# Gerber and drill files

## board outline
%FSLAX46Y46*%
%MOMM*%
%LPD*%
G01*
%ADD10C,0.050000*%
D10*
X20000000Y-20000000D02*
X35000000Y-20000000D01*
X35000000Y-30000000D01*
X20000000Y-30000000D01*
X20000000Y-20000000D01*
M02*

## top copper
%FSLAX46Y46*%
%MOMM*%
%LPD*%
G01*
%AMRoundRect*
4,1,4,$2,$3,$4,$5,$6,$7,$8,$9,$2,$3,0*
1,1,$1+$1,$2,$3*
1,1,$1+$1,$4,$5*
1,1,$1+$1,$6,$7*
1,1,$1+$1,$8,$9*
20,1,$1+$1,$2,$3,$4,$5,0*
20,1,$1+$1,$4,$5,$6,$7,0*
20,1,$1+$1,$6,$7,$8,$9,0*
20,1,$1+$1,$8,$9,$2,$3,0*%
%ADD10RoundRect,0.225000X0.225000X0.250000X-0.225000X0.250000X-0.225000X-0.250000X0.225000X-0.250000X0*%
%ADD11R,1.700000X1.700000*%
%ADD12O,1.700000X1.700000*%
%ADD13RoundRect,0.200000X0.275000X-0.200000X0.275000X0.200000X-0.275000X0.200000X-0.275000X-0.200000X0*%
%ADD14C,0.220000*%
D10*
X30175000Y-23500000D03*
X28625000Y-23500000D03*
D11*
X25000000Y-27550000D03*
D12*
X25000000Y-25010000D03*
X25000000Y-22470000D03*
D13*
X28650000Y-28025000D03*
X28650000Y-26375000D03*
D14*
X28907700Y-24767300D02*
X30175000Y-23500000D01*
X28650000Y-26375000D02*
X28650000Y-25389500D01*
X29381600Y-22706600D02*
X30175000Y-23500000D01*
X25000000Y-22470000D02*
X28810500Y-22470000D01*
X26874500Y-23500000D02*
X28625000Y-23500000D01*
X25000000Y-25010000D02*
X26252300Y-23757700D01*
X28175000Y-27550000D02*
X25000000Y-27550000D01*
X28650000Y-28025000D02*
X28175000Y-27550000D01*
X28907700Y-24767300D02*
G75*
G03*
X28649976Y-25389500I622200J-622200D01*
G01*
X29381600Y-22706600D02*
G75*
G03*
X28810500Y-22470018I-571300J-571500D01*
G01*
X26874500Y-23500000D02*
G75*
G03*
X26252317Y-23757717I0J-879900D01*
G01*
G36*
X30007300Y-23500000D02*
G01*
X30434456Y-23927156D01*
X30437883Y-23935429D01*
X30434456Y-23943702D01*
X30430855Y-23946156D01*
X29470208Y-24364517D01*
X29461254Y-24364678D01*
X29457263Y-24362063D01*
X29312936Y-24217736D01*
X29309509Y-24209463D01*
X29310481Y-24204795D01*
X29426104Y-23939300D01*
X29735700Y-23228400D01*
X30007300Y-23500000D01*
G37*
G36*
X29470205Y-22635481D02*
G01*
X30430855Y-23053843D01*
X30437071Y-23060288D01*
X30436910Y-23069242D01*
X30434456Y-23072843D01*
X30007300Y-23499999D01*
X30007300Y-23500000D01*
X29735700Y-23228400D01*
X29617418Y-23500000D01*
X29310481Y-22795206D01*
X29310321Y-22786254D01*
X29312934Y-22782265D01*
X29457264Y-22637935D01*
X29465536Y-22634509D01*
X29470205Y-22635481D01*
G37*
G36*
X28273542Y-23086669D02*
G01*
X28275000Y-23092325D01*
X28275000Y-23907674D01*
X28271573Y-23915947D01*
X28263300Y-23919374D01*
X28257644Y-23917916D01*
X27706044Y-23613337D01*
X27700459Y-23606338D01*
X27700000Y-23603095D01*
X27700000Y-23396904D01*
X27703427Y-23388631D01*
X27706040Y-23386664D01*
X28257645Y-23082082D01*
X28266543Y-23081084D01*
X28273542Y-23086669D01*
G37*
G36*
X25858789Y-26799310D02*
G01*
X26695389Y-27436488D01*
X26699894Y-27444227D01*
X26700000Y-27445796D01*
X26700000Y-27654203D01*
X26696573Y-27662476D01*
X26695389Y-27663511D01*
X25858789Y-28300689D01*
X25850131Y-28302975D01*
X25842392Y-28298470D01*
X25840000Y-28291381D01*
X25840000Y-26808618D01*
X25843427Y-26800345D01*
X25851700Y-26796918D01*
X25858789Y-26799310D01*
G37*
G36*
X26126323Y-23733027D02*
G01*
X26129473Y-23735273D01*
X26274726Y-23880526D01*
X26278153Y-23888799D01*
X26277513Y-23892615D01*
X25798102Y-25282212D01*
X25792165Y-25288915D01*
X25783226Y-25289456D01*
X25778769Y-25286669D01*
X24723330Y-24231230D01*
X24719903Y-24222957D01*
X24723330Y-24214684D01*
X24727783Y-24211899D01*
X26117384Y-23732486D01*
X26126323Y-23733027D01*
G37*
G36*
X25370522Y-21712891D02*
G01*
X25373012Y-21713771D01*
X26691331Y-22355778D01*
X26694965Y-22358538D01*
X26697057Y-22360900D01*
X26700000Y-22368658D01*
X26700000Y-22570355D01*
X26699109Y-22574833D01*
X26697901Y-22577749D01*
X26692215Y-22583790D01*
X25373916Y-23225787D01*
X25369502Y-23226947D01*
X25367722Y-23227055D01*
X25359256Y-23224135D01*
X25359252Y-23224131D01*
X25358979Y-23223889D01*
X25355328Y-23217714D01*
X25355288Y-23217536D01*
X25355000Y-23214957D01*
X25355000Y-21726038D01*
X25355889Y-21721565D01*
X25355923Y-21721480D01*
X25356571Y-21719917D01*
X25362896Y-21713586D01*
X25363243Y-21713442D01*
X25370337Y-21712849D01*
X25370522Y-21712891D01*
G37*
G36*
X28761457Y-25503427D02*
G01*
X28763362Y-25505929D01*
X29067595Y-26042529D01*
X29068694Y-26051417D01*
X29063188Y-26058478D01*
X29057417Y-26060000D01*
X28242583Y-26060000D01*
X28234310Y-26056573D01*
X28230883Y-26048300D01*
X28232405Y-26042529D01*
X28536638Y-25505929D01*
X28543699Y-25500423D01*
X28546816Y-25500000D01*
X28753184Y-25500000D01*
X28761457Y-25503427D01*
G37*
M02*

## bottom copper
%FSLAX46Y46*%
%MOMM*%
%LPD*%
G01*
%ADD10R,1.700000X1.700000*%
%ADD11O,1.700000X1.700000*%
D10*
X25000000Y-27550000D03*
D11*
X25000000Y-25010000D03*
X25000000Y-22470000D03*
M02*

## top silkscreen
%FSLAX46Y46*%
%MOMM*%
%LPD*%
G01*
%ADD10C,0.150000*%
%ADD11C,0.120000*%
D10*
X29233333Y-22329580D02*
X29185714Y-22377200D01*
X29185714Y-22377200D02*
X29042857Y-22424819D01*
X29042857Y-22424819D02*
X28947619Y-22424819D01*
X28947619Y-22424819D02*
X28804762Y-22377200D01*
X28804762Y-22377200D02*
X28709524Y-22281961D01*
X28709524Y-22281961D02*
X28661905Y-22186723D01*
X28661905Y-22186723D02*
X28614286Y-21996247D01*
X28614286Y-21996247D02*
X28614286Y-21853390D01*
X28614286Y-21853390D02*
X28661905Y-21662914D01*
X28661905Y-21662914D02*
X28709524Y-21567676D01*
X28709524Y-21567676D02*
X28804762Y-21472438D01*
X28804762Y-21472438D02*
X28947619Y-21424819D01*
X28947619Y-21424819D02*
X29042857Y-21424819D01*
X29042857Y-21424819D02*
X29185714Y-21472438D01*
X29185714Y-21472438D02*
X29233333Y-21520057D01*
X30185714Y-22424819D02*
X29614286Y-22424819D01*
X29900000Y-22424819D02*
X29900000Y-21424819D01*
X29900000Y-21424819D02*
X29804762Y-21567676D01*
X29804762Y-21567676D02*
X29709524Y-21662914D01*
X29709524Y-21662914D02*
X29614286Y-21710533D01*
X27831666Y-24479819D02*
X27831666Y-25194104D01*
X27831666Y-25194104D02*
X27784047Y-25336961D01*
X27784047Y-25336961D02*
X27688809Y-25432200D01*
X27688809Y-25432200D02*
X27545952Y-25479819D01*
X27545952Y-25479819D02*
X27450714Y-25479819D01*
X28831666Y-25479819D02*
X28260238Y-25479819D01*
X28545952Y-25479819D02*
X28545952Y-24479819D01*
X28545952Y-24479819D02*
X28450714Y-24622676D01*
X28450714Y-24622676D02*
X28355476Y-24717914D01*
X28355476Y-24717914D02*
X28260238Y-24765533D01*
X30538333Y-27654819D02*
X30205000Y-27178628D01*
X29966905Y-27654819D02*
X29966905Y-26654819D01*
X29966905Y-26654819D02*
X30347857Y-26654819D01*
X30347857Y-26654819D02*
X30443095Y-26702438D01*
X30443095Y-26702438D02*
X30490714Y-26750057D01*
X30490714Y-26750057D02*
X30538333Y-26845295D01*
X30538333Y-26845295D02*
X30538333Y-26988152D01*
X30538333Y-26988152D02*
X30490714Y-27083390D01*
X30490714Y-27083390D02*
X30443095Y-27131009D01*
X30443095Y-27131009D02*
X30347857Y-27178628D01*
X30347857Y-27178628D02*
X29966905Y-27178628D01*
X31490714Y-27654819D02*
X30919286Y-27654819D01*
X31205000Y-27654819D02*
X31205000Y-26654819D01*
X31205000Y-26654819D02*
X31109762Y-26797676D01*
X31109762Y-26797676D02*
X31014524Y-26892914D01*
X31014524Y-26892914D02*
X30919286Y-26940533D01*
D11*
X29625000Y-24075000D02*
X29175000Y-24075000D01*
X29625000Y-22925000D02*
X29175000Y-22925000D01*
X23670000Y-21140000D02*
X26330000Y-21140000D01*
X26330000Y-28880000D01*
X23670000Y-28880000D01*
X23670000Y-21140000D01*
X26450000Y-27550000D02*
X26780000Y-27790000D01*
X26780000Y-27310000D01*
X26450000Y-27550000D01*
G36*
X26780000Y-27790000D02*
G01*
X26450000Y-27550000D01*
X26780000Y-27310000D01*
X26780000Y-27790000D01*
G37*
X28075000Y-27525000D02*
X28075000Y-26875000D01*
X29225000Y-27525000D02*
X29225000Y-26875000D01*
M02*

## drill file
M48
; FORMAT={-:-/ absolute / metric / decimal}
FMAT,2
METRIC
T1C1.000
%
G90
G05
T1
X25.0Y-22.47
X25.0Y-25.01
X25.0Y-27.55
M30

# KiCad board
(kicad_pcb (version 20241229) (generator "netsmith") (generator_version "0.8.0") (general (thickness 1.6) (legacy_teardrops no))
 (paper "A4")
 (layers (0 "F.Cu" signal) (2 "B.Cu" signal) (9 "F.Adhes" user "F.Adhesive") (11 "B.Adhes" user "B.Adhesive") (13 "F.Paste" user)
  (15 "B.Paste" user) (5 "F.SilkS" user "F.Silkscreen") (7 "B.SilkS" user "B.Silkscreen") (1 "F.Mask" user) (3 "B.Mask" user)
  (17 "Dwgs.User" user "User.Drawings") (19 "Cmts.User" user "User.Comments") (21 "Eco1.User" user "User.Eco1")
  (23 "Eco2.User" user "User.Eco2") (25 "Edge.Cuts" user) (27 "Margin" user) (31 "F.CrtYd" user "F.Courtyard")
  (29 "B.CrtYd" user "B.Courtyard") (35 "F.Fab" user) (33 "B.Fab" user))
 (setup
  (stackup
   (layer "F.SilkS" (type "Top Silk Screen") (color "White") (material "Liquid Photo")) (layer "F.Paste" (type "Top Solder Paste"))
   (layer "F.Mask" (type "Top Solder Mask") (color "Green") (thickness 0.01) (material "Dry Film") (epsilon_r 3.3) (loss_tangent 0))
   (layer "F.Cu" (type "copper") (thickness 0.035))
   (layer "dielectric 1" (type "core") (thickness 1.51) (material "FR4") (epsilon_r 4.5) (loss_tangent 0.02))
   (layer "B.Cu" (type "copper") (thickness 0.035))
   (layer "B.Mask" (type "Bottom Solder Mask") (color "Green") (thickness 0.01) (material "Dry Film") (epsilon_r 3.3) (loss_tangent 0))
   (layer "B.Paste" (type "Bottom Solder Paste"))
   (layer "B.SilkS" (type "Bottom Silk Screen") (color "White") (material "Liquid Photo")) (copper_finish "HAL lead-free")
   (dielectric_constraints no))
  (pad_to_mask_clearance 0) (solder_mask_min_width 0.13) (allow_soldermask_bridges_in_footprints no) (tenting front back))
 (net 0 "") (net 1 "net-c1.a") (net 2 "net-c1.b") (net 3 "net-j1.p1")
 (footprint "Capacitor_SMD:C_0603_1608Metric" (layer "F.Cu") (at 29.4 23.5 180)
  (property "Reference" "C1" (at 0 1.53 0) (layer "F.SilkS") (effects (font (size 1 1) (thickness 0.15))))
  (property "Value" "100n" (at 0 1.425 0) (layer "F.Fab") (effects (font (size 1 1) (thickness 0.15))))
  (pad "1" smd roundrect (at -0.775 0 180) (size 0.9 0.95) (layers "F.Cu" "F.Mask" "F.Paste") (roundrect_rratio 0.25) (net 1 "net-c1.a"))
  (pad "2" smd roundrect (at 0.775 0 180) (size 0.9 0.95) (layers "F.Cu" "F.Mask" "F.Paste") (roundrect_rratio 0.25) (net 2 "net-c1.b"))
  (fp_line (start -0.225 -0.575) (end 0.225 -0.575) (stroke (width 0.12) (type solid)) (layer "F.SilkS"))
  (fp_line (start -0.225 0.575) (end 0.225 0.575) (stroke (width 0.12) (type solid)) (layer "F.SilkS")))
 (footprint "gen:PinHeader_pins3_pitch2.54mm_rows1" (layer "F.Cu") (at 25 27.55 180)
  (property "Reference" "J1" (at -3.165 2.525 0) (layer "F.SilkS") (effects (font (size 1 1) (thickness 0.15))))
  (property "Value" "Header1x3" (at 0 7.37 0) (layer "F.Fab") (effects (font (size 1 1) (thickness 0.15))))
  (pad "1" thru_hole rect (at 0 0 180) (size 1.7 1.7) (drill 1) (layers "*.Cu" "*.Mask") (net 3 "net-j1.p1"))
  (pad "2" thru_hole oval (at 0 2.54 180) (size 1.7 1.7) (drill 1) (layers "*.Cu" "*.Mask") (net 2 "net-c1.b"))
  (pad "3" thru_hole oval (at 0 5.08 180) (size 1.7 1.7) (drill 1) (layers "*.Cu" "*.Mask") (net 1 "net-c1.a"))
  (fp_rect (start -1.33 -1.33) (end 1.33 6.41) (stroke (width 0.12) (type solid)) (fill no) (layer "F.SilkS"))
  (fp_poly (pts (xy -1.45 0) (xy -1.78 -0.24) (xy -1.78 0.24)) (stroke (width 0.12) (type solid)) (fill solid) (layer "F.SilkS")))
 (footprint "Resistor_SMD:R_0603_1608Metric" (layer "F.Cu") (at 28.65 27.2 90)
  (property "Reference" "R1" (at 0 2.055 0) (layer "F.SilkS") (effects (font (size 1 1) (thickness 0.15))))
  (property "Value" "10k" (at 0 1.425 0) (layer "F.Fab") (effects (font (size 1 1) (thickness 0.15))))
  (pad "1" smd roundrect (at -0.825 0 90) (size 0.8 0.95) (layers "F.Cu" "F.Mask" "F.Paste") (roundrect_rratio 0.25) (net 3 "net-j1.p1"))
  (pad "2" smd roundrect (at 0.825 0 90) (size 0.8 0.95) (layers "F.Cu" "F.Mask" "F.Paste") (roundrect_rratio 0.25) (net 1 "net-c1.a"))
  (fp_line (start -0.325 -0.575) (end 0.325 -0.575) (stroke (width 0.12) (type solid)) (layer "F.SilkS"))
  (fp_line (start -0.325 0.575) (end 0.325 0.575) (stroke (width 0.12) (type solid)) (layer "F.SilkS")))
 (segment (start 28.9077 24.7673) (end 30.175 23.5) (width 0.22) (layer "F.Cu") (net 1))
 (segment (start 28.65 26.375) (end 28.65 25.3895) (width 0.22) (layer "F.Cu") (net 1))
 (segment (start 29.3816 22.7066) (end 30.175 23.5) (width 0.22) (layer "F.Cu") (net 1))
 (segment (start 25 22.47) (end 28.8105 22.47) (width 0.22) (layer "F.Cu") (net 1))
 (segment (start 26.8745 23.5) (end 28.625 23.5) (width 0.22) (layer "F.Cu") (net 2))
 (segment (start 25 25.01) (end 26.2523 23.7577) (width 0.22) (layer "F.Cu") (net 2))
 (segment (start 28.175 27.55) (end 25 27.55) (width 0.22) (layer "F.Cu") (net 3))
 (segment (start 28.65 28.025) (end 28.175 27.55) (width 0.22) (layer "F.Cu") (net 3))
 (arc (start 28.9077 24.7673) (mid 28.717 25.0527) (end 28.65 25.3895) (width 0.22) (layer "F.Cu") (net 1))
 (arc (start 29.3816 22.7066) (mid 29.1195 22.5315) (end 28.8105 22.47) (width 0.22) (layer "F.Cu") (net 1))
 (arc (start 26.8745 23.5) (mid 26.5377 23.567) (end 26.2523 23.7577) (width 0.22) (layer "F.Cu") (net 2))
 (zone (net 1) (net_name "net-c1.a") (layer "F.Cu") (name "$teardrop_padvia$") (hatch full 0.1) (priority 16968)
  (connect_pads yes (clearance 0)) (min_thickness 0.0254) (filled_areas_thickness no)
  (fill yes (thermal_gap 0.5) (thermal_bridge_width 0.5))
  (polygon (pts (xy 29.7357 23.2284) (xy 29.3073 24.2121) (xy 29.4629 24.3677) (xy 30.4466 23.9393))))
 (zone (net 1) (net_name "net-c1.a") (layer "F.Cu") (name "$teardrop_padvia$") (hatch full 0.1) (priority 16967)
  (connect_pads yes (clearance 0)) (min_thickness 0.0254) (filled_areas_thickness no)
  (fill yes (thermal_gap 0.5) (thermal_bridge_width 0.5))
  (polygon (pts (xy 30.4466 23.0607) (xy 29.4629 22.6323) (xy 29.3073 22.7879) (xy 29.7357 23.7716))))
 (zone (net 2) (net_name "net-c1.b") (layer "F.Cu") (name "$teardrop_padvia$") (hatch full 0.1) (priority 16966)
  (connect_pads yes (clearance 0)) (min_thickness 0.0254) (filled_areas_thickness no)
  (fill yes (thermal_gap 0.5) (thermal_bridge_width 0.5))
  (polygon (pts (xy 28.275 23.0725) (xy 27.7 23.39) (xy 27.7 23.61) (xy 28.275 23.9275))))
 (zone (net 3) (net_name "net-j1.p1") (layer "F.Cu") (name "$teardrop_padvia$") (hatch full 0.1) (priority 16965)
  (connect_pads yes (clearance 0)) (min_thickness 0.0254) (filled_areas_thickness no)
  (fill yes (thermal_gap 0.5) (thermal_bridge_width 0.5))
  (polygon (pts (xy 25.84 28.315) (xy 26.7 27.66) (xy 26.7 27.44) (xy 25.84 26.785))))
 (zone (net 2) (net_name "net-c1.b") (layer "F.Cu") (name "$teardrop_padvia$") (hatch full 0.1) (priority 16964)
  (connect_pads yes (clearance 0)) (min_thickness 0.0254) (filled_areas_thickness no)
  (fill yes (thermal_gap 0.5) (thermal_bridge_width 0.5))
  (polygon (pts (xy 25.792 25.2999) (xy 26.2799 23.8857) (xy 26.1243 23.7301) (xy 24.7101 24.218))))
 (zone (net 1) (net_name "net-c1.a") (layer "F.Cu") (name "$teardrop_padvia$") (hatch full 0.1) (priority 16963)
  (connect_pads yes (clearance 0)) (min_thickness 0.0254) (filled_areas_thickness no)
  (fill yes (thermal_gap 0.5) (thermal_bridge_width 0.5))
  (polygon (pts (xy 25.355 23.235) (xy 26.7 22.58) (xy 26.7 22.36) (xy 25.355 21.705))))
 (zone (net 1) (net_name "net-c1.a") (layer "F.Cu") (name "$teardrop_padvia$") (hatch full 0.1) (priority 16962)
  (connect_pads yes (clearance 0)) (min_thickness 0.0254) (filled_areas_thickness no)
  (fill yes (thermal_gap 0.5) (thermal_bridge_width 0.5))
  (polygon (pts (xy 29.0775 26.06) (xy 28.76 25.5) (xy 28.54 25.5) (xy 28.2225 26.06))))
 (gr_rect (start 20 20) (end 35 30) (stroke (width 0.05) (type default)) (fill no) (layer "Edge.Cuts")))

